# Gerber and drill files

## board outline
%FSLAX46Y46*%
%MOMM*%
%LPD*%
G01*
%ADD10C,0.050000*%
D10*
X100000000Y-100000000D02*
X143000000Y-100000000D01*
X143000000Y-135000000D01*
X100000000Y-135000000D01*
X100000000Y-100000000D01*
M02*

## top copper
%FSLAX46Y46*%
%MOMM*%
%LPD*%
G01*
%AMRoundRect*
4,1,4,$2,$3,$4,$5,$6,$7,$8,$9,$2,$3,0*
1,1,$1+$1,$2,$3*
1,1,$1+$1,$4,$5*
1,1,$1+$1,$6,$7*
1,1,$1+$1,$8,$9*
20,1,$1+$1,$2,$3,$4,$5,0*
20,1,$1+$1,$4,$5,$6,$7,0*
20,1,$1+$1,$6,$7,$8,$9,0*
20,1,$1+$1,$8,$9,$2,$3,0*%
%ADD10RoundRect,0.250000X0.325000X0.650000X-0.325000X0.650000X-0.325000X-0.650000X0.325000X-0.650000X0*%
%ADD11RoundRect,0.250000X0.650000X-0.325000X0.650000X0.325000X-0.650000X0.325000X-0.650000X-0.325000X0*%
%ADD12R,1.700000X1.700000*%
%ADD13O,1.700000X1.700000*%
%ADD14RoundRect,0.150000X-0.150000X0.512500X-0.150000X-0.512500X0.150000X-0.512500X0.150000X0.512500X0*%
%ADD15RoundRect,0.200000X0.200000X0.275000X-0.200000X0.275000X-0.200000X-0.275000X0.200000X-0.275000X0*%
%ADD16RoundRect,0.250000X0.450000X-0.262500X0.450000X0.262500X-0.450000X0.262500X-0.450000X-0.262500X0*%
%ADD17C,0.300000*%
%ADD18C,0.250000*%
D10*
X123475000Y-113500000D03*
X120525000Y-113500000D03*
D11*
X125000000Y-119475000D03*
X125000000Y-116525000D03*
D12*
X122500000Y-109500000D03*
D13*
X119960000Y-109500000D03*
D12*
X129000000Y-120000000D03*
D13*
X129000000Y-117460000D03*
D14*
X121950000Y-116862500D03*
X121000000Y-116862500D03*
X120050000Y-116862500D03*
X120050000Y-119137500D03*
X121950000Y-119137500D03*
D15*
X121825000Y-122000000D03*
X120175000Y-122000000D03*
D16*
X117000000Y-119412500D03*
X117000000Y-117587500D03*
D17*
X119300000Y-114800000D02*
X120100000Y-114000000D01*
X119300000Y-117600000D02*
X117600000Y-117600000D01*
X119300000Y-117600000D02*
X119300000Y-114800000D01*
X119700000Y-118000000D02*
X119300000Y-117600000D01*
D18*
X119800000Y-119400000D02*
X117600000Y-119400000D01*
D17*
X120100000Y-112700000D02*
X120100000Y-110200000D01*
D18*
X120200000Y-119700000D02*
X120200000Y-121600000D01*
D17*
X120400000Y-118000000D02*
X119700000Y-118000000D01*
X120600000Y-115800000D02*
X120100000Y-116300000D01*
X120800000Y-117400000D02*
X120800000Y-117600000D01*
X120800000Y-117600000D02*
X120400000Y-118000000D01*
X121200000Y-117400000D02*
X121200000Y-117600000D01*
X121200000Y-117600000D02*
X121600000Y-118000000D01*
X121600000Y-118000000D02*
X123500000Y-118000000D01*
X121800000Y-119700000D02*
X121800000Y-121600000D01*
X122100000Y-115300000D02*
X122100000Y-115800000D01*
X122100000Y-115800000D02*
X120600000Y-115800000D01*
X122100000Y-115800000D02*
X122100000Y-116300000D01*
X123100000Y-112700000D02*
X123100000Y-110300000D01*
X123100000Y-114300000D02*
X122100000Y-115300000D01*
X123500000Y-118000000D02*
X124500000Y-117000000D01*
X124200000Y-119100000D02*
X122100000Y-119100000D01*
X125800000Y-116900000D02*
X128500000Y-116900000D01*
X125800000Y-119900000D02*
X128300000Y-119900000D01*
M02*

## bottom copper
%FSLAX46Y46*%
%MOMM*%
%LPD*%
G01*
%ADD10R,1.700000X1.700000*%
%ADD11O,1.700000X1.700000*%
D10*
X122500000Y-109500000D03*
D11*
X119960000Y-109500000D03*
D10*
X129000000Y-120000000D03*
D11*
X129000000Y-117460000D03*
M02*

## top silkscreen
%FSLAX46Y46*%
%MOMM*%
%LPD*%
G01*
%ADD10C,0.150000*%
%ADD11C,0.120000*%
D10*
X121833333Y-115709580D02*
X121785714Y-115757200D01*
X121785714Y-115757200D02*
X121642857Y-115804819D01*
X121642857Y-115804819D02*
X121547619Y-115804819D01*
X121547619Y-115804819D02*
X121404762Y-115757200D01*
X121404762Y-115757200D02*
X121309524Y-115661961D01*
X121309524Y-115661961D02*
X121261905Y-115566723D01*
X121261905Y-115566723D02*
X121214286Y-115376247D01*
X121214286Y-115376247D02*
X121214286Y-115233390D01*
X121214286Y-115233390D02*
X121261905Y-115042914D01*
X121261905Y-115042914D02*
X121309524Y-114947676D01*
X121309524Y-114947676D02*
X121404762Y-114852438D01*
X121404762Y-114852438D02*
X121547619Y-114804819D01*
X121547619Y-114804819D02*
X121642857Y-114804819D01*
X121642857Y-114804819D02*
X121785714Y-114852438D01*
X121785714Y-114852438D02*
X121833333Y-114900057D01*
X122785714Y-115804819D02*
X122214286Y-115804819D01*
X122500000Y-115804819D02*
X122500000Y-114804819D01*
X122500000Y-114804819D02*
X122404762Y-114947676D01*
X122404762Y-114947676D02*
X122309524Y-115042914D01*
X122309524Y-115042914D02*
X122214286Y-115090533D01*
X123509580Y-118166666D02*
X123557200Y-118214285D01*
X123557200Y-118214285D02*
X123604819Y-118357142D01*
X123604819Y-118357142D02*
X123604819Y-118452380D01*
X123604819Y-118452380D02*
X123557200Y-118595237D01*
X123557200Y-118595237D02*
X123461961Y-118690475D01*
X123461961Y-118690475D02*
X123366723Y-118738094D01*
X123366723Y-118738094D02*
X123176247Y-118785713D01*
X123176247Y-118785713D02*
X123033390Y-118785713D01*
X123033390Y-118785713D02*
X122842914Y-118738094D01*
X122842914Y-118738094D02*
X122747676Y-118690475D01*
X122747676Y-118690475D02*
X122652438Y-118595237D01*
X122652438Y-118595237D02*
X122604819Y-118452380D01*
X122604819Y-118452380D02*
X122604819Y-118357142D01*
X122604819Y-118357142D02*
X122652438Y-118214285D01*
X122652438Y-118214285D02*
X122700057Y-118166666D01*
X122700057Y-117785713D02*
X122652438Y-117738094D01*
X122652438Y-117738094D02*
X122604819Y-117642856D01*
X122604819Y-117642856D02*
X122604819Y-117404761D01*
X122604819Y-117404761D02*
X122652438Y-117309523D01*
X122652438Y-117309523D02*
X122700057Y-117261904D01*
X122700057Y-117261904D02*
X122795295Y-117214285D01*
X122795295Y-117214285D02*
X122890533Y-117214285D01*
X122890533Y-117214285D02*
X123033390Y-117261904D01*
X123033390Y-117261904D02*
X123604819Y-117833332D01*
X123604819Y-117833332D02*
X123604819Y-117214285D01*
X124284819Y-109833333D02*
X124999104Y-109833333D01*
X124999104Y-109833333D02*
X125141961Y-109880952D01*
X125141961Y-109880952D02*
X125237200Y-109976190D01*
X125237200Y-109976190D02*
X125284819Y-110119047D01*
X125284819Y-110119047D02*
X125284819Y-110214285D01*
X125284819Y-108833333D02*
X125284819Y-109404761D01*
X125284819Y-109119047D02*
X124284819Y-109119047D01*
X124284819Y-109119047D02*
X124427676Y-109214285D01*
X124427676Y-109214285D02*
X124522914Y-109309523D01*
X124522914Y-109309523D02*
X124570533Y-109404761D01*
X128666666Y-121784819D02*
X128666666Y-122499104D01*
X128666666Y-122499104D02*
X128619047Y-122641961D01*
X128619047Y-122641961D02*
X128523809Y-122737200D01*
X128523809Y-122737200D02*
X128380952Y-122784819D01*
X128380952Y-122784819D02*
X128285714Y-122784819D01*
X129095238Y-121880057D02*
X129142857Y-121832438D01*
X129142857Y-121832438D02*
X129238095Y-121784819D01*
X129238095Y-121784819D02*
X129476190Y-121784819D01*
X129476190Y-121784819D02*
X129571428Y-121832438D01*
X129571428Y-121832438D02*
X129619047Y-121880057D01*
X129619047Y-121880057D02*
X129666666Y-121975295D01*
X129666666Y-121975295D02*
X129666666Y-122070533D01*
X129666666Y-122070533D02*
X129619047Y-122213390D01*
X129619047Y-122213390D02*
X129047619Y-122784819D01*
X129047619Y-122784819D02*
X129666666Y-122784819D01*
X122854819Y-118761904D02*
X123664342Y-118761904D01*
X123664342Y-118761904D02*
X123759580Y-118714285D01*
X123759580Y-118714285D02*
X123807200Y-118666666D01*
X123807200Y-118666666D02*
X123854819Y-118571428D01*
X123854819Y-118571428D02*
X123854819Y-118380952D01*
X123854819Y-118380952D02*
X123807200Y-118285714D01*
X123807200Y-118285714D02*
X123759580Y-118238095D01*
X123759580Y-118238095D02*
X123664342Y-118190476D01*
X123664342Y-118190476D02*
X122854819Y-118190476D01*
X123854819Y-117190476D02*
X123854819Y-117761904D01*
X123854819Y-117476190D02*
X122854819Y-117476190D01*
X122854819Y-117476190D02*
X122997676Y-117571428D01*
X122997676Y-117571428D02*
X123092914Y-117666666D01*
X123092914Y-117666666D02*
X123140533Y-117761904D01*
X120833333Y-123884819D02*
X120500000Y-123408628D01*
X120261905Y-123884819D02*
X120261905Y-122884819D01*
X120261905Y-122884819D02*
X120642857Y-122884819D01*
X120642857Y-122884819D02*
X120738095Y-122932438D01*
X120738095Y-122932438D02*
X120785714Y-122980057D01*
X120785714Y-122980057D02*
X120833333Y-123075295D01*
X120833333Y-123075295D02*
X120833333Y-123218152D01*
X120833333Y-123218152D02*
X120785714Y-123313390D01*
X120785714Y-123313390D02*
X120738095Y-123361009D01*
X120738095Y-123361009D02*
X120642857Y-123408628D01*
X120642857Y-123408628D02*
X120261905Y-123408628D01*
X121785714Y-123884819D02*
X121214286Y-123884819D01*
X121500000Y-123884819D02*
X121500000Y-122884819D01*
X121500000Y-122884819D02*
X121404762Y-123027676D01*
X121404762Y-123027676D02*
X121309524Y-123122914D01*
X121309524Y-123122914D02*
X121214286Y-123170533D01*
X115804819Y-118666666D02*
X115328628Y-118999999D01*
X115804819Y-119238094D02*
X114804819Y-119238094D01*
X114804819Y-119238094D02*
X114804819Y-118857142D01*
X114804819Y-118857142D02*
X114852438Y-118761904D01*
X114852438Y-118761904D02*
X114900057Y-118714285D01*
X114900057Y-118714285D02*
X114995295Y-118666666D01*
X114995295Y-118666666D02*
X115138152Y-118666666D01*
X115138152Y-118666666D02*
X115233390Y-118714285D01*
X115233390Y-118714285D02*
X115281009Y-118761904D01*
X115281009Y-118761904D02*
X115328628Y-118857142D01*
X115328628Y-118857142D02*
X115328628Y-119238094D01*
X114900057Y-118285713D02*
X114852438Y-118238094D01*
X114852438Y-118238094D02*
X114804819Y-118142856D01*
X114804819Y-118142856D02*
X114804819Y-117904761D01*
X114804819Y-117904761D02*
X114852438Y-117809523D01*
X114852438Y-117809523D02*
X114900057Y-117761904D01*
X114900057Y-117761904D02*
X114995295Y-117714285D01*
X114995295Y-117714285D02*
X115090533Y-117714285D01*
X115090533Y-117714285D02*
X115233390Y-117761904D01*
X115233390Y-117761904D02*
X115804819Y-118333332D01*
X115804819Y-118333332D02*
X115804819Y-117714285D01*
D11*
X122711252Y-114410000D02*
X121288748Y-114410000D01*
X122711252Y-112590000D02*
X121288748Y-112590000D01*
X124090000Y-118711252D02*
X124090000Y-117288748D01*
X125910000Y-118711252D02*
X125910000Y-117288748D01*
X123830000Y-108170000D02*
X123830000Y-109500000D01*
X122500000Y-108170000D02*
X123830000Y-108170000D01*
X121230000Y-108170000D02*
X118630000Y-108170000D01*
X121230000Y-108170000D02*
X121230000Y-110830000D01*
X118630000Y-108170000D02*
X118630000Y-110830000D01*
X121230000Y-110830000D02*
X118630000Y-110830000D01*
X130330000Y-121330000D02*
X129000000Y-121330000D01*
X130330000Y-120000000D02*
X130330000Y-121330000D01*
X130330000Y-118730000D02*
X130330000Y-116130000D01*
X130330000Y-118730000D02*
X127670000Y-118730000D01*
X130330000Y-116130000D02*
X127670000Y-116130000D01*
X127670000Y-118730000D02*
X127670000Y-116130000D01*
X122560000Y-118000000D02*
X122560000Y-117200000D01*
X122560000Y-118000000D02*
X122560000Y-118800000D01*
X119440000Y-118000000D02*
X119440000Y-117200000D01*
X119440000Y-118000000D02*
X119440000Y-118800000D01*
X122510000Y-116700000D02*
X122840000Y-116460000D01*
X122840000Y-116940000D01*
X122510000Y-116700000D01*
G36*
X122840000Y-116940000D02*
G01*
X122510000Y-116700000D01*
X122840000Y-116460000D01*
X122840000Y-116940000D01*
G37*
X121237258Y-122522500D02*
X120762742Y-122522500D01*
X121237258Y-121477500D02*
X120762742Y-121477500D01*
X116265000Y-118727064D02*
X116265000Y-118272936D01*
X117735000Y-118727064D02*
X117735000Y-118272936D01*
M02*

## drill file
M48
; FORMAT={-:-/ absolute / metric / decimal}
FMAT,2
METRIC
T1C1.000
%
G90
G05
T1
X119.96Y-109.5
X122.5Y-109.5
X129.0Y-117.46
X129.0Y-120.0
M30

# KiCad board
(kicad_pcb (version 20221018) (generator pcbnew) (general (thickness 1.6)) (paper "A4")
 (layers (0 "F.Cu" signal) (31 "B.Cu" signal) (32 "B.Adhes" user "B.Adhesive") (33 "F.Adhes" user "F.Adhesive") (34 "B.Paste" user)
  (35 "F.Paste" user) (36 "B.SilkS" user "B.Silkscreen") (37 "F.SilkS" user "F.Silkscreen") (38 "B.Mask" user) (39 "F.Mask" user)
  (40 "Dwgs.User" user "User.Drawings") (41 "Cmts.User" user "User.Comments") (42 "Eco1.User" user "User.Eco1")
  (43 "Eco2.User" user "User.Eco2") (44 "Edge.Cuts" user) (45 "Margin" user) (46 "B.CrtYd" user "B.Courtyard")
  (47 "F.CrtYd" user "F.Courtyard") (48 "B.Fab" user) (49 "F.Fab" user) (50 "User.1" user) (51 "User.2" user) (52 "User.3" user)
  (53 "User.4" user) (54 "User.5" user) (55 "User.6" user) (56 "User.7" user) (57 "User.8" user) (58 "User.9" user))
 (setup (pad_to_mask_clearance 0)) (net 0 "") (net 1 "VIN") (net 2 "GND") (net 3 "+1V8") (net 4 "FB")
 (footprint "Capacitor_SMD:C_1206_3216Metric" (layer "F.Cu") (at 122 113.5 180)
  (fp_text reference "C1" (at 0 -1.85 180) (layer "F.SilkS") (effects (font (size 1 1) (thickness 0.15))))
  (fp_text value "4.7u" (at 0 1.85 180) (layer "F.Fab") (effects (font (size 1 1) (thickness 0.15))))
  (fp_line (start -0.711252 -0.91) (end 0.711252 -0.91) (stroke (width 0.12) (type solid)) (layer "F.SilkS"))
  (fp_line (start -0.711252 0.91) (end 0.711252 0.91) (stroke (width 0.12) (type solid)) (layer "F.SilkS"))
  (pad "1" smd roundrect (at -1.475 0 180) (size 1.15 1.8) (layers "F.Cu" "F.Paste" "F.Mask") (roundrect_rratio 0.217391) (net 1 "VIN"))
  (pad "2" smd roundrect (at 1.475 0 180) (size 1.15 1.8) (layers "F.Cu" "F.Paste" "F.Mask") (roundrect_rratio 0.217391) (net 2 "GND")))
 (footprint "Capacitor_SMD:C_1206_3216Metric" (layer "F.Cu") (at 125 118 90)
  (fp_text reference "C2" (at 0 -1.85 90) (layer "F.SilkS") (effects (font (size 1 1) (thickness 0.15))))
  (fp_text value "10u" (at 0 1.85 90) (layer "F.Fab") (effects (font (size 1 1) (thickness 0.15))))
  (fp_line (start -0.711252 -0.91) (end 0.711252 -0.91) (stroke (width 0.12) (type solid)) (layer "F.SilkS"))
  (fp_line (start -0.711252 0.91) (end 0.711252 0.91) (stroke (width 0.12) (type solid)) (layer "F.SilkS"))
  (pad "1" smd roundrect (at -1.475 0 90) (size 1.15 1.8) (layers "F.Cu" "F.Paste" "F.Mask") (roundrect_rratio 0.217391) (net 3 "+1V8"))
  (pad "2" smd roundrect (at 1.475 0 90) (size 1.15 1.8) (layers "F.Cu" "F.Paste" "F.Mask") (roundrect_rratio 0.217391) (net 2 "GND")))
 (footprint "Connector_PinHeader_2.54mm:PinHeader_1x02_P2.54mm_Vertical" (layer "F.Cu") (at 122.5 109.5 -90)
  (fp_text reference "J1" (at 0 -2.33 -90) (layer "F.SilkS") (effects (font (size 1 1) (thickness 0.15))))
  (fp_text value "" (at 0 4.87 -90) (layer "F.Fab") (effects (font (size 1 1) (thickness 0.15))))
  (fp_line (start -1.33 -1.33) (end 0 -1.33) (stroke (width 0.12) (type solid)) (layer "F.SilkS"))
  (fp_line (start -1.33 0) (end -1.33 -1.33) (stroke (width 0.12) (type solid)) (layer "F.SilkS"))
  (fp_line (start -1.33 1.27) (end -1.33 3.87) (stroke (width 0.12) (type solid)) (layer "F.SilkS"))
  (fp_line (start -1.33 1.27) (end 1.33 1.27) (stroke (width 0.12) (type solid)) (layer "F.SilkS"))
  (fp_line (start -1.33 3.87) (end 1.33 3.87) (stroke (width 0.12) (type solid)) (layer "F.SilkS"))
  (fp_line (start 1.33 1.27) (end 1.33 3.87) (stroke (width 0.12) (type solid)) (layer "F.SilkS"))
  (pad "1" thru_hole rect (at 0 0 270) (size 1.7 1.7) (drill 1) (layers "*.Cu" "*.Mask") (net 1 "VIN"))
  (pad "2" thru_hole oval (at 0 2.54 270) (size 1.7 1.7) (drill 1) (layers "*.Cu" "*.Mask") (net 2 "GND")))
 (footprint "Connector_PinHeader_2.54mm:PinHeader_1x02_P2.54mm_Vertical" (layer "F.Cu") (at 129 120 180)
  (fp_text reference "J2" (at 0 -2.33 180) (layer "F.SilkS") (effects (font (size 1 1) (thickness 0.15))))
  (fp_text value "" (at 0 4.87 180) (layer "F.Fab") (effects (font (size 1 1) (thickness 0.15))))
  (fp_line (start -1.33 -1.33) (end 0 -1.33) (stroke (width 0.12) (type solid)) (layer "F.SilkS"))
  (fp_line (start -1.33 0) (end -1.33 -1.33) (stroke (width 0.12) (type solid)) (layer "F.SilkS"))
  (fp_line (start -1.33 1.27) (end -1.33 3.87) (stroke (width 0.12) (type solid)) (layer "F.SilkS"))
  (fp_line (start -1.33 1.27) (end 1.33 1.27) (stroke (width 0.12) (type solid)) (layer "F.SilkS"))
  (fp_line (start -1.33 3.87) (end 1.33 3.87) (stroke (width 0.12) (type solid)) (layer "F.SilkS"))
  (fp_line (start 1.33 1.27) (end 1.33 3.87) (stroke (width 0.12) (type solid)) (layer "F.SilkS"))
  (pad "1" thru_hole rect (at 0 0 180) (size 1.7 1.7) (drill 1) (layers "*.Cu" "*.Mask") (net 3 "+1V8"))
  (pad "2" thru_hole oval (at 0 2.54 180) (size 1.7 1.7) (drill 1) (layers "*.Cu" "*.Mask") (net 2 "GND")))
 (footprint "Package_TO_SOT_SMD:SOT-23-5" (layer "F.Cu") (at 121 118 -90)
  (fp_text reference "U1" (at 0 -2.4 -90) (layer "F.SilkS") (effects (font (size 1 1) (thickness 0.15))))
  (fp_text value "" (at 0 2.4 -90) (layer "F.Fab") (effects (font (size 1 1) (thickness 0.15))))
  (fp_line (start 0 -1.56) (end -0.8 -1.56) (stroke (width 0.12) (type solid)) (layer "F.SilkS"))
  (fp_line (start 0 -1.56) (end 0.8 -1.56) (stroke (width 0.12) (type solid)) (layer "F.SilkS"))
  (fp_line (start 0 1.56) (end -0.8 1.56) (stroke (width 0.12) (type solid)) (layer "F.SilkS"))
  (fp_line (start 0 1.56) (end 0.8 1.56) (stroke (width 0.12) (type solid)) (layer "F.SilkS"))
  (fp_poly
   (pts (xy -1.3 -1.51) (xy -1.54 -1.84) (xy -1.06 -1.84) (xy -1.3 -1.51)) (stroke (width 0.12) (type solid)) (fill solid) (layer "F.SilkS"))
  (pad "1" smd roundrect (at -1.1375 -0.95 270) (size 1.325 0.6) (layers "F.Cu" "F.Paste" "F.Mask") (roundrect_rratio 0.25) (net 1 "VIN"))
  (pad "2" smd roundrect (at -1.1375 0 270) (size 1.325 0.6) (layers "F.Cu" "F.Paste" "F.Mask") (roundrect_rratio 0.25) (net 2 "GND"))
  (pad "3" smd roundrect (at -1.1375 0.95 270) (size 1.325 0.6) (layers "F.Cu" "F.Paste" "F.Mask") (roundrect_rratio 0.25) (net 1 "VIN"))
  (pad "4" smd roundrect (at 1.1375 0.95 270) (size 1.325 0.6) (layers "F.Cu" "F.Paste" "F.Mask") (roundrect_rratio 0.25) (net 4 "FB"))
  (pad "5" smd roundrect (at 1.1375 -0.95 270) (size 1.325 0.6) (layers "F.Cu" "F.Paste" "F.Mask") (roundrect_rratio 0.25) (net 3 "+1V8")))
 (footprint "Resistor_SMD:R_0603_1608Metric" (layer "F.Cu") (at 121 122 180)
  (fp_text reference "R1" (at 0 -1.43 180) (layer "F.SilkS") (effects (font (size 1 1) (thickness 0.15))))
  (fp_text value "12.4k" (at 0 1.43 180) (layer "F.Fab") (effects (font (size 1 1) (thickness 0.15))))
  (fp_line (start -0.237258 -0.5225) (end 0.237258 -0.5225) (stroke (width 0.12) (type solid)) (layer "F.SilkS"))
  (fp_line (start -0.237258 0.5225) (end 0.237258 0.5225) (stroke (width 0.12) (type solid)) (layer "F.SilkS"))
  (pad "1" smd roundrect (at -0.825 0 180) (size 0.8 0.95) (layers "F.Cu" "F.Paste" "F.Mask") (roundrect_rratio 0.25) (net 3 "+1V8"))
  (pad "2" smd roundrect (at 0.825 0 180) (size 0.8 0.95) (layers "F.Cu" "F.Paste" "F.Mask") (roundrect_rratio 0.25) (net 4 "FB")))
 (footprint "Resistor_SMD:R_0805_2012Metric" (layer "F.Cu") (at 117 118.5 90)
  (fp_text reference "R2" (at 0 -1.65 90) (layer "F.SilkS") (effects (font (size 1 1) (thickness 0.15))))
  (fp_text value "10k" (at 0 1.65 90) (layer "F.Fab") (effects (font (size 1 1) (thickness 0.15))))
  (fp_line (start -0.227064 -0.735) (end 0.227064 -0.735) (stroke (width 0.12) (type solid)) (layer "F.SilkS"))
  (fp_line (start -0.227064 0.735) (end 0.227064 0.735) (stroke (width 0.12) (type solid)) (layer "F.SilkS"))
  (pad "1" smd roundrect (at -0.9125 0 90) (size 1.025 1.4) (layers "F.Cu" "F.Paste" "F.Mask") (roundrect_rratio 0.243902) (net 4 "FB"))
  (pad "2" smd roundrect (at 0.9125 0 90) (size 1.025 1.4) (layers "F.Cu" "F.Paste" "F.Mask") (roundrect_rratio 0.243902) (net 2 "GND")))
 (gr_rect (start 100 100) (end 143 135) (stroke (width 0.05) (type default)) (fill none) (layer "Edge.Cuts"))
 (segment (start 119.3 114.8) (end 120.1 114) (width 0.3) (layer "F.Cu") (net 2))
 (segment (start 119.3 117.6) (end 117.6 117.6) (width 0.3) (layer "F.Cu") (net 2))
 (segment (start 119.3 117.6) (end 119.3 114.8) (width 0.3) (layer "F.Cu") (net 2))
 (segment (start 119.7 118) (end 119.3 117.6) (width 0.3) (layer "F.Cu") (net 2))
 (segment (start 119.8 119.4) (end 117.6 119.4) (width 0.25) (layer "F.Cu") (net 4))
 (segment (start 120.1 112.7) (end 120.1 110.2) (width 0.3) (layer "F.Cu") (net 2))
 (segment (start 120.2 119.7) (end 120.2 121.6) (width 0.25) (layer "F.Cu") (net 4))
 (segment (start 120.4 118) (end 119.7 118) (width 0.3) (layer "F.Cu") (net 2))
 (segment (start 120.6 115.8) (end 120.1 116.3) (width 0.3) (layer "F.Cu") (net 1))
 (segment (start 120.8 117.4) (end 120.8 117.6) (width 0.3) (layer "F.Cu") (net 2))
 (segment (start 120.8 117.6) (end 120.4 118) (width 0.3) (layer "F.Cu") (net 2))
 (segment (start 121.2 117.4) (end 121.2 117.6) (width 0.3) (layer "F.Cu") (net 2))
 (segment (start 121.2 117.6) (end 121.6 118) (width 0.3) (layer "F.Cu") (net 2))
 (segment (start 121.6 118) (end 123.5 118) (width 0.3) (layer "F.Cu") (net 2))
 (segment (start 121.8 119.7) (end 121.8 121.6) (width 0.3) (layer "F.Cu") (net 3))
 (segment (start 122.1 115.3) (end 122.1 115.8) (width 0.3) (layer "F.Cu") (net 1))
 (segment (start 122.1 115.8) (end 120.6 115.8) (width 0.3) (layer "F.Cu") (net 1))
 (segment (start 122.1 115.8) (end 122.1 116.3) (width 0.3) (layer "F.Cu") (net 1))
 (segment (start 123.1 112.7) (end 123.1 110.3) (width 0.3) (layer "F.Cu") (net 1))
 (segment (start 123.1 114.3) (end 122.1 115.3) (width 0.3) (layer "F.Cu") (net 1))
 (segment (start 123.5 118) (end 124.5 117) (width 0.3) (layer "F.Cu") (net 2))
 (segment (start 124.2 119.1) (end 122.1 119.1) (width 0.3) (layer "F.Cu") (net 3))
 (segment (start 125.8 116.9) (end 128.5 116.9) (width 0.3) (layer "F.Cu") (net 2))
 (segment (start 125.8 119.9) (end 128.3 119.9) (width 0.3) (layer "F.Cu") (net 3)))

